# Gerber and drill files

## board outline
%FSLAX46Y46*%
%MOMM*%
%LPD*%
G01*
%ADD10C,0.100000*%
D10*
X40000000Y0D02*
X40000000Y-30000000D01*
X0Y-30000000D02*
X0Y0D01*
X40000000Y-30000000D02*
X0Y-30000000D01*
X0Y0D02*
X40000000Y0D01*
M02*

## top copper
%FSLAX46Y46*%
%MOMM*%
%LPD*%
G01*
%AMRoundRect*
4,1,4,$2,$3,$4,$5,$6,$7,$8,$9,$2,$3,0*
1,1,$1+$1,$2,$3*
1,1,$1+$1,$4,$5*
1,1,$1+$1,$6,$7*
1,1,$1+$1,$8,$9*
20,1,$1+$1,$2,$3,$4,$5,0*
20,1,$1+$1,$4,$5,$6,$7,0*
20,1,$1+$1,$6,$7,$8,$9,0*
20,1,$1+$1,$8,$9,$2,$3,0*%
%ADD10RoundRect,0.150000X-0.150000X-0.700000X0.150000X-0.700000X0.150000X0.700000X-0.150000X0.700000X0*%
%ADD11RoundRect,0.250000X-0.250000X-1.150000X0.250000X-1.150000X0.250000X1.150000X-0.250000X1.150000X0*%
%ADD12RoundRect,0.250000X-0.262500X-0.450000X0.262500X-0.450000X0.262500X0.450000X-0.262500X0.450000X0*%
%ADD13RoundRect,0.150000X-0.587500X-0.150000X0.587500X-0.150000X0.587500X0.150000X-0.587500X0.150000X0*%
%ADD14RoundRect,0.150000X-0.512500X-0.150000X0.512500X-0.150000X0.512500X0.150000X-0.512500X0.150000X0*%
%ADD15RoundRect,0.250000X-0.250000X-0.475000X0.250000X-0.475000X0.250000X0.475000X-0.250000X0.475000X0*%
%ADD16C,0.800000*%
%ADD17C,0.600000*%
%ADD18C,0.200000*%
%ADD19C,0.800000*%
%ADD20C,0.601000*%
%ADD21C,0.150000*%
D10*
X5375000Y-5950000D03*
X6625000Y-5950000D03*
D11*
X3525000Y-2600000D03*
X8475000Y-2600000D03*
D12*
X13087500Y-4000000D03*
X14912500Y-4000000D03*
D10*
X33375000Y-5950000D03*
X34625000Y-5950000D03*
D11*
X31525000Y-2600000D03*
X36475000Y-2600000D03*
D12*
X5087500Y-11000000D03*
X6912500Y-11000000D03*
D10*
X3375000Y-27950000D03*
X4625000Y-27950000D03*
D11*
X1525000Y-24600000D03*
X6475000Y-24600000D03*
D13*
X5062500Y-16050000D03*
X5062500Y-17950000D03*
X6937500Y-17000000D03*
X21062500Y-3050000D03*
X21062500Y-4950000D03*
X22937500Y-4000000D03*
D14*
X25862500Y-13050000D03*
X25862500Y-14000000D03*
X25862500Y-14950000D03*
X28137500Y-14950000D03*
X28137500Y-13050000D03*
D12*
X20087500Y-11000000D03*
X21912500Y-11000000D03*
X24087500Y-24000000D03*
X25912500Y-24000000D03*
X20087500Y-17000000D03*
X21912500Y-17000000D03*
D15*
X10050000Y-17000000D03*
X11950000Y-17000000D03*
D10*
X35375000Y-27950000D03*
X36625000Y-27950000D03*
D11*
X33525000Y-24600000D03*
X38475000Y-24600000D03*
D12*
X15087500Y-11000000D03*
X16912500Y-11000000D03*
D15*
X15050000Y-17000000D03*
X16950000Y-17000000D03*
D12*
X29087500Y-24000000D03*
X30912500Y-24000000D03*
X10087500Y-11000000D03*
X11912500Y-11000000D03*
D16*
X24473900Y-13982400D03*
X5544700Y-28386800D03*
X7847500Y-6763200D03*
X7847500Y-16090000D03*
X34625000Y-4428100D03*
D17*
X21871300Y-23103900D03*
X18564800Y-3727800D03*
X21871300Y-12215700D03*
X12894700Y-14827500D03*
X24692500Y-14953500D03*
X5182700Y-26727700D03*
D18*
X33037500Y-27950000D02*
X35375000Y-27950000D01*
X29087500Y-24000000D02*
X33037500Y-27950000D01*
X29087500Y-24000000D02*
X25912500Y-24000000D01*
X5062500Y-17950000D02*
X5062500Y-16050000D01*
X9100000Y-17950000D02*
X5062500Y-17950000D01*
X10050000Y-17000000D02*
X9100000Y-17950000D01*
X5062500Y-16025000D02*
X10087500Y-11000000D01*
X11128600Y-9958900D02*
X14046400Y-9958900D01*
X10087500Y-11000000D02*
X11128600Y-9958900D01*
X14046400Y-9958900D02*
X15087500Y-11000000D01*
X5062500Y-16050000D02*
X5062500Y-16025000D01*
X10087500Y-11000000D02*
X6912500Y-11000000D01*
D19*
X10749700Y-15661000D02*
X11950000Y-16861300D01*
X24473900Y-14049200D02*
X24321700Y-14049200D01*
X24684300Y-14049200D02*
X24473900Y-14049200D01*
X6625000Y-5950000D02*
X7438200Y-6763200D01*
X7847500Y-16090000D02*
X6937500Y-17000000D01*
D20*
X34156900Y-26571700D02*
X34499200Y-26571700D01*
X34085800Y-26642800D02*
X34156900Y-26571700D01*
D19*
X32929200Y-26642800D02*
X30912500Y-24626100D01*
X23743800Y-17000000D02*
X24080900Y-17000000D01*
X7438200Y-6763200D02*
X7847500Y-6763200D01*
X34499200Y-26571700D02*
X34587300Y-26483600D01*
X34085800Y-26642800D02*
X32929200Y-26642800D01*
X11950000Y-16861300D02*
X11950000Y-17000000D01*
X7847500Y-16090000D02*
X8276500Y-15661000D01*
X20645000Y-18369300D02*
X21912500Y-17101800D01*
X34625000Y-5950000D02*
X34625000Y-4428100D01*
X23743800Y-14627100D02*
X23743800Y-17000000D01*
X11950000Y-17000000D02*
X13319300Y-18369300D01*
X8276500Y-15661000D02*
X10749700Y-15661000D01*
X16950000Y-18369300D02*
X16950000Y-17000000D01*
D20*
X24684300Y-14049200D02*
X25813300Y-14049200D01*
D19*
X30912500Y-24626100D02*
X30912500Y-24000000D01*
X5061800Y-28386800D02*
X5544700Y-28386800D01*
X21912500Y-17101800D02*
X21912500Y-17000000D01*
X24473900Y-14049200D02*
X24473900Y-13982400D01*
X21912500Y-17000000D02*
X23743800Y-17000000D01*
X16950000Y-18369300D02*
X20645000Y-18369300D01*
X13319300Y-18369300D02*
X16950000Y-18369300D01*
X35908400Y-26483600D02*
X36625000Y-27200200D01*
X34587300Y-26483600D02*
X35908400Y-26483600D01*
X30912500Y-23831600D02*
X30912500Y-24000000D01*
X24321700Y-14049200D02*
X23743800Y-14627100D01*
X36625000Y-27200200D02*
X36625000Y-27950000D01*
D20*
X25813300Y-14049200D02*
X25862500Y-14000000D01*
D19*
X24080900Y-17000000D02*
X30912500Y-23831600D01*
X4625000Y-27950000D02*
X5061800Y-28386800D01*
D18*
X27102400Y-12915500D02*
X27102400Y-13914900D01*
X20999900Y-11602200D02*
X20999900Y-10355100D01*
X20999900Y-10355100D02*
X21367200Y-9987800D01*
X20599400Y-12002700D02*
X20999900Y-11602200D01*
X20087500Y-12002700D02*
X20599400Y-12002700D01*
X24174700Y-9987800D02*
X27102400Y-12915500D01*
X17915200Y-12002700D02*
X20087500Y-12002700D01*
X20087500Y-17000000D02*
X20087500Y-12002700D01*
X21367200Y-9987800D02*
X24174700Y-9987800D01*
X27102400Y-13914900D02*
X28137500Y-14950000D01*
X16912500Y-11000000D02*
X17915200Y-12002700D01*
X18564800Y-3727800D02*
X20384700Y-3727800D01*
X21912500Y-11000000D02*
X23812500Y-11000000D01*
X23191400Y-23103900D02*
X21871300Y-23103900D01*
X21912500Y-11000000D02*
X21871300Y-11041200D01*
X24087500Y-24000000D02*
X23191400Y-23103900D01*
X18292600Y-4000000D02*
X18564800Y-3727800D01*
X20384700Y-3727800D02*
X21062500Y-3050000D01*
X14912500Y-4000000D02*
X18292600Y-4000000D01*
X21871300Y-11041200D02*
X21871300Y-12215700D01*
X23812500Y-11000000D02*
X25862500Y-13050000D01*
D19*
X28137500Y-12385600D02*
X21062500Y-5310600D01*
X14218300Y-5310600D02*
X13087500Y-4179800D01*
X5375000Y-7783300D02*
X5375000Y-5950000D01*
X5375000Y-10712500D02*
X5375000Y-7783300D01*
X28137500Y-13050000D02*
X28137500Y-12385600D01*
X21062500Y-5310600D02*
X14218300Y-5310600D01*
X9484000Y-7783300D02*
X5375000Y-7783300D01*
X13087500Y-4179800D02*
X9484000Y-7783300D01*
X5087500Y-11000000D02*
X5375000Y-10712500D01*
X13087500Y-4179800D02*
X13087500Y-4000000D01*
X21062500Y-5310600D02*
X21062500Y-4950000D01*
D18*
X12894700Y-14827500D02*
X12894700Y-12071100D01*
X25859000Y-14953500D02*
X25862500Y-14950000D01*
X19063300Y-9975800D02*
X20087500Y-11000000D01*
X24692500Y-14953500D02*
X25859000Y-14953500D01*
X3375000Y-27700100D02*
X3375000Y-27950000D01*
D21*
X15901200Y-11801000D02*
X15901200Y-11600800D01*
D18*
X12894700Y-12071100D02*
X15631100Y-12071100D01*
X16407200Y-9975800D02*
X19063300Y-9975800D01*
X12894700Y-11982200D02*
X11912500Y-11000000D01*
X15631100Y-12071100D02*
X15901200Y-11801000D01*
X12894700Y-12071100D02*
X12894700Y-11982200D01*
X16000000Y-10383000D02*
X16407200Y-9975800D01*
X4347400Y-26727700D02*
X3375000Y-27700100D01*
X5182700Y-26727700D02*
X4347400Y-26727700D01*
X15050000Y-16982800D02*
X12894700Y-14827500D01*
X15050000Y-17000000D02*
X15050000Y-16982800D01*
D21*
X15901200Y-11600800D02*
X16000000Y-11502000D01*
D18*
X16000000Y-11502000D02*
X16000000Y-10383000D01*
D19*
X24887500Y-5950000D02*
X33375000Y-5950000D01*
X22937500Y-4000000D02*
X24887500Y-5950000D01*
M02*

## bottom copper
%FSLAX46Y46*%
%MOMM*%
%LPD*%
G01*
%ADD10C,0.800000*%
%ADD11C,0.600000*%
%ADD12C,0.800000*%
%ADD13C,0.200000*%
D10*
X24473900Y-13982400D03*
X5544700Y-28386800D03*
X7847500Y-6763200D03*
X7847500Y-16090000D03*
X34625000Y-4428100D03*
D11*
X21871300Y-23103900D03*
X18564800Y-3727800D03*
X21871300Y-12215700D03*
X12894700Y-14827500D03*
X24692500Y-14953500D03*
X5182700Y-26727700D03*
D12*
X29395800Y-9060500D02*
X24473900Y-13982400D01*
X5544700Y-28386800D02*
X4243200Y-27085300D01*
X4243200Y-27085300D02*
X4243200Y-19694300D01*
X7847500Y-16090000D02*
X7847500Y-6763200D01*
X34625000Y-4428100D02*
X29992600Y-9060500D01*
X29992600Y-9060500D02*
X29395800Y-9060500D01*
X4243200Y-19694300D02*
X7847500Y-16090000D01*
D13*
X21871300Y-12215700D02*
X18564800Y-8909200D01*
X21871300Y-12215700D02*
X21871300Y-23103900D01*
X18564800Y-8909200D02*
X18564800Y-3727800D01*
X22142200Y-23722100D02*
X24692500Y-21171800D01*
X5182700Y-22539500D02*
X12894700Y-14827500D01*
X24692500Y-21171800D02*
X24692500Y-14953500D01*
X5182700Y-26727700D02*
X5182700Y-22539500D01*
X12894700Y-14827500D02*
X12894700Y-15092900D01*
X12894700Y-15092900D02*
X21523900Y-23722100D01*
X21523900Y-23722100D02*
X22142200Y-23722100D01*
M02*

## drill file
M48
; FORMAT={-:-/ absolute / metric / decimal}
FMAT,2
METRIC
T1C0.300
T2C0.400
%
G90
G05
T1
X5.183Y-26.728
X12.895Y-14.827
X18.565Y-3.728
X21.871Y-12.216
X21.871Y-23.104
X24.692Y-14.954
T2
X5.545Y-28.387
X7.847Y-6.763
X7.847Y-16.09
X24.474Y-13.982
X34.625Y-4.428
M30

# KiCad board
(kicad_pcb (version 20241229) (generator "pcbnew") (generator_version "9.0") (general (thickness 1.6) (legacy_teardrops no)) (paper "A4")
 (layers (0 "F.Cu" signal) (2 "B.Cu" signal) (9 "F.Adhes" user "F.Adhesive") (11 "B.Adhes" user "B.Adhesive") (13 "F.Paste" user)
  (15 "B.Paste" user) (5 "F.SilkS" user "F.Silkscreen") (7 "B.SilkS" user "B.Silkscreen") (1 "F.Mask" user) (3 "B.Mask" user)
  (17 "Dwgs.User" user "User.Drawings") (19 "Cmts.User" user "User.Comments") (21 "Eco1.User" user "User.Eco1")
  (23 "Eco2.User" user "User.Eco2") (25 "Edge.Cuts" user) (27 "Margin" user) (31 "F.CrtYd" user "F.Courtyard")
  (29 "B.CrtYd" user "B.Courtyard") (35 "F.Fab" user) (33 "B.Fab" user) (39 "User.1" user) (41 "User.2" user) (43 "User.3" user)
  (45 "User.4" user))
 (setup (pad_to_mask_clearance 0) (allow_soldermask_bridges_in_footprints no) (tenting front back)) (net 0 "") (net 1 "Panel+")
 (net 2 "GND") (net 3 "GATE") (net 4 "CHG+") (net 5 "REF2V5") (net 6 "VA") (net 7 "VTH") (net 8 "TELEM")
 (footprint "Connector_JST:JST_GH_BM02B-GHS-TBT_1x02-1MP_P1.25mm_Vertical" (layer "F.Cu") (at 6 4)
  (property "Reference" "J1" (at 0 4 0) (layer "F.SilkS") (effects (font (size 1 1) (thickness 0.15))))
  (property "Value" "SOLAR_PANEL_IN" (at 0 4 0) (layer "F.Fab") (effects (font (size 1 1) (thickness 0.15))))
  (pad "1" smd roundrect (at -0.625 1.95) (size 0.6 1.7) (layers "F.Cu" "F.Mask" "F.Paste") (roundrect_rratio 0.25) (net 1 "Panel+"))
  (pad "2" smd roundrect (at 0.625 1.95) (size 0.6 1.7) (layers "F.Cu" "F.Mask" "F.Paste") (roundrect_rratio 0.25) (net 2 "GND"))
  (pad "MP" smd roundrect (at -2.475 -1.4) (size 1 2.8) (layers "F.Cu" "F.Mask" "F.Paste") (roundrect_rratio 0.25))
  (pad "MP" smd roundrect (at 2.475 -1.4) (size 1 2.8) (layers "F.Cu" "F.Mask" "F.Paste") (roundrect_rratio 0.25)))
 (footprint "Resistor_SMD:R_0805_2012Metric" (layer "F.Cu") (at 14 4)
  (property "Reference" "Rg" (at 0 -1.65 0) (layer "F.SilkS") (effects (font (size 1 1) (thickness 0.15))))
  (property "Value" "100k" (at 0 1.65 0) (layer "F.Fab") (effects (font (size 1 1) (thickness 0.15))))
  (pad "1" smd roundrect (at -0.9125 0) (size 1.025 1.4) (layers "F.Cu" "F.Mask" "F.Paste") (roundrect_rratio 0.243902) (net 1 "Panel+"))
  (pad "2" smd roundrect (at 0.9125 0) (size 1.025 1.4) (layers "F.Cu" "F.Mask" "F.Paste") (roundrect_rratio 0.243902) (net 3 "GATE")))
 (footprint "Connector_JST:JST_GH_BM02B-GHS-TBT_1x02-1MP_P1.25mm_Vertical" (layer "F.Cu") (at 34 4)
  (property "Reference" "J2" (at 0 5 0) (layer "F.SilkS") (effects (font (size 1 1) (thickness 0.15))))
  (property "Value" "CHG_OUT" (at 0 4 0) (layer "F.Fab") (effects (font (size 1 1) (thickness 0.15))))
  (pad "1" smd roundrect (at -0.625 1.95) (size 0.6 1.7) (layers "F.Cu" "F.Mask" "F.Paste") (roundrect_rratio 0.25) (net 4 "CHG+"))
  (pad "2" smd roundrect (at 0.625 1.95) (size 0.6 1.7) (layers "F.Cu" "F.Mask" "F.Paste") (roundrect_rratio 0.25) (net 2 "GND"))
  (pad "MP" smd roundrect (at -2.475 -1.4) (size 1 2.8) (layers "F.Cu" "F.Mask" "F.Paste") (roundrect_rratio 0.25))
  (pad "MP" smd roundrect (at 2.475 -1.4) (size 1 2.8) (layers "F.Cu" "F.Mask" "F.Paste") (roundrect_rratio 0.25)))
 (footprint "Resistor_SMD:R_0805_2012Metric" (layer "F.Cu") (at 6 11)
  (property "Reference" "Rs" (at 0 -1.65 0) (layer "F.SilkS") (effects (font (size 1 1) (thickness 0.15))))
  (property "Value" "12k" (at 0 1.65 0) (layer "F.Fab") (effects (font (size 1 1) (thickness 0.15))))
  (pad "1" smd roundrect (at -0.9125 0) (size 1.025 1.4) (layers "F.Cu" "F.Mask" "F.Paste") (roundrect_rratio 0.243902) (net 1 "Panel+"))
  (pad "2" smd roundrect (at 0.9125 0) (size 1.025 1.4) (layers "F.Cu" "F.Mask" "F.Paste") (roundrect_rratio 0.243902) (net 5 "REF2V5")))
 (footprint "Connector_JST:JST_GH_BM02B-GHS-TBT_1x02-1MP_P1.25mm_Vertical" (layer "F.Cu") (at 4 26)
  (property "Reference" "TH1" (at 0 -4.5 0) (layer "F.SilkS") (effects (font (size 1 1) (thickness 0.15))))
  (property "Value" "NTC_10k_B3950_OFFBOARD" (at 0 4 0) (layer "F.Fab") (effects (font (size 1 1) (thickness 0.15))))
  (pad "1" smd roundrect (at -0.625 1.95) (size 0.6 1.7) (layers "F.Cu" "F.Mask" "F.Paste") (roundrect_rratio 0.25) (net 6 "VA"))
  (pad "2" smd roundrect (at 0.625 1.95) (size 0.6 1.7) (layers "F.Cu" "F.Mask" "F.Paste") (roundrect_rratio 0.25) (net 2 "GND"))
  (pad "MP" smd roundrect (at -2.475 -1.4) (size 1 2.8) (layers "F.Cu" "F.Mask" "F.Paste") (roundrect_rratio 0.25))
  (pad "MP" smd roundrect (at 2.475 -1.4) (size 1 2.8) (layers "F.Cu" "F.Mask" "F.Paste") (roundrect_rratio 0.25)))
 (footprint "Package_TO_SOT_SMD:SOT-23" (layer "F.Cu") (at 6 17)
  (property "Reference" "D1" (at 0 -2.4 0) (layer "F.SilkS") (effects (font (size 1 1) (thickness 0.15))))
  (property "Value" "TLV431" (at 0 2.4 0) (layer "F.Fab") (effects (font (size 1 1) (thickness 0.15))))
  (pad "1" smd roundrect (at -0.9375 -0.95) (size 1.475 0.6) (layers "F.Cu" "F.Mask" "F.Paste") (roundrect_rratio 0.25) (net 5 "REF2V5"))
  (pad "2" smd roundrect (at -0.9375 0.95) (size 1.475 0.6) (layers "F.Cu" "F.Mask" "F.Paste") (roundrect_rratio 0.25) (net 5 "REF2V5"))
  (pad "3" smd roundrect (at 0.9375 0) (size 1.475 0.6) (layers "F.Cu" "F.Mask" "F.Paste") (roundrect_rratio 0.25) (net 2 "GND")))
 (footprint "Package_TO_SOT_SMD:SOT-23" (layer "F.Cu") (at 22 4)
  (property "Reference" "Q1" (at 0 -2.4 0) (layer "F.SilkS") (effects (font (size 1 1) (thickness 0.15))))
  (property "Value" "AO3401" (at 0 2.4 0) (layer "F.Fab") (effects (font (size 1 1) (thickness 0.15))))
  (pad "1" smd roundrect (at -0.9375 -0.95) (size 1.475 0.6) (layers "F.Cu" "F.Mask" "F.Paste") (roundrect_rratio 0.25) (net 3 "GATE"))
  (pad "2" smd roundrect (at -0.9375 0.95) (size 1.475 0.6) (layers "F.Cu" "F.Mask" "F.Paste") (roundrect_rratio 0.25) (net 1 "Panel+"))
  (pad "3" smd roundrect (at 0.9375 0) (size 1.475 0.6) (layers "F.Cu" "F.Mask" "F.Paste") (roundrect_rratio 0.25) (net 4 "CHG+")))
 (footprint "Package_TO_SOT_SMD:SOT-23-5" (layer "F.Cu") (at 27 14)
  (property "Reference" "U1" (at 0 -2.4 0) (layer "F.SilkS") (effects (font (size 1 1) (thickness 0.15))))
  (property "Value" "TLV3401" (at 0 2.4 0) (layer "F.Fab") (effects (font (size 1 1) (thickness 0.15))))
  (pad "1" smd roundrect (at -1.1375 -0.95) (size 1.325 0.6) (layers "F.Cu" "F.Mask" "F.Paste") (roundrect_rratio 0.25) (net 3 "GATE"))
  (pad "2" smd roundrect (at -1.1375 0) (size 1.325 0.6) (layers "F.Cu" "F.Mask" "F.Paste") (roundrect_rratio 0.25) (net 2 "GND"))
  (pad "3" smd roundrect (at -1.1375 0.95) (size 1.325 0.6) (layers "F.Cu" "F.Mask" "F.Paste") (roundrect_rratio 0.25) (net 6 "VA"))
  (pad "4" smd roundrect (at 1.1375 0.95) (size 1.325 0.6) (layers "F.Cu" "F.Mask" "F.Paste") (roundrect_rratio 0.25) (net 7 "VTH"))
  (pad "5" smd roundrect (at 1.1375 -0.95) (size 1.325 0.6) (layers "F.Cu" "F.Mask" "F.Paste") (roundrect_rratio 0.25) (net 1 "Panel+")))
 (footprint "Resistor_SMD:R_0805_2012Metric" (layer "F.Cu") (at 21 11)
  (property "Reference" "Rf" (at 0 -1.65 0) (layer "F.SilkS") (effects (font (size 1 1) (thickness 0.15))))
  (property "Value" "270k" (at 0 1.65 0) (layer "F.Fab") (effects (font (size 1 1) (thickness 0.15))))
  (pad "1" smd roundrect (at -0.9125 0) (size 1.025 1.4) (layers "F.Cu" "F.Mask" "F.Paste") (roundrect_rratio 0.243902) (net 6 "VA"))
  (pad "2" smd roundrect (at 0.9125 0) (size 1.025 1.4) (layers "F.Cu" "F.Mask" "F.Paste") (roundrect_rratio 0.243902) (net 3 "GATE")))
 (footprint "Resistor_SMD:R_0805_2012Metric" (layer "F.Cu") (at 25 24)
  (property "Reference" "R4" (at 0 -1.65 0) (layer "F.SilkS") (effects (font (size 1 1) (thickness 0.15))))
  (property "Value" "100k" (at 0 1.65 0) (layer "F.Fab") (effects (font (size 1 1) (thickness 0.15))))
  (pad "1" smd roundrect (at -0.9125 0) (size 1.025 1.4) (layers "F.Cu" "F.Mask" "F.Paste") (roundrect_rratio 0.243902) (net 3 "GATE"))
  (pad "2" smd roundrect (at 0.9125 0) (size 1.025 1.4) (layers "F.Cu" "F.Mask" "F.Paste") (roundrect_rratio 0.243902) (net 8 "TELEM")))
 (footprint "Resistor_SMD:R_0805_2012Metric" (layer "F.Cu") (at 21 17)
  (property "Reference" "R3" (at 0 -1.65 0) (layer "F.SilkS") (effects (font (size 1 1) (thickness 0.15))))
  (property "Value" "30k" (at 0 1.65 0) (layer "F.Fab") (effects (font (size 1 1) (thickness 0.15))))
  (pad "1" smd roundrect (at -0.9125 0) (size 1.025 1.4) (layers "F.Cu" "F.Mask" "F.Paste") (roundrect_rratio 0.243902) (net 7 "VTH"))
  (pad "2" smd roundrect (at 0.9125 0) (size 1.025 1.4) (layers "F.Cu" "F.Mask" "F.Paste") (roundrect_rratio 0.243902) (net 2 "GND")))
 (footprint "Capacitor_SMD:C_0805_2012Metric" (layer "F.Cu") (at 11 17)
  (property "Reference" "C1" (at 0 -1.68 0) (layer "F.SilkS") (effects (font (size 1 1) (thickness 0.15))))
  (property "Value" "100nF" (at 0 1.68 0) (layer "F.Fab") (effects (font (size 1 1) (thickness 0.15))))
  (pad "1" smd roundrect (at -0.95 0) (size 1 1.45) (layers "F.Cu" "F.Mask" "F.Paste") (roundrect_rratio 0.25) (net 5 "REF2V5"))
  (pad "2" smd roundrect (at 0.95 0) (size 1 1.45) (layers "F.Cu" "F.Mask" "F.Paste") (roundrect_rratio 0.25) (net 2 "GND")))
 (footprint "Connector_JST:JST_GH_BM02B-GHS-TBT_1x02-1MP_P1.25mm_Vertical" (layer "F.Cu") (at 36 26)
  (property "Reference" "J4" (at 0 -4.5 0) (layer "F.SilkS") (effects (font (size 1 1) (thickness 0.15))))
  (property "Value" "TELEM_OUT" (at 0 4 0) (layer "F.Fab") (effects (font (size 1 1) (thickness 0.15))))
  (pad "1" smd roundrect (at -0.625 1.95) (size 0.6 1.7) (layers "F.Cu" "F.Mask" "F.Paste") (roundrect_rratio 0.25) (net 8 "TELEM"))
  (pad "2" smd roundrect (at 0.625 1.95) (size 0.6 1.7) (layers "F.Cu" "F.Mask" "F.Paste") (roundrect_rratio 0.25) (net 2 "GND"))
  (pad "MP" smd roundrect (at -2.475 -1.4) (size 1 2.8) (layers "F.Cu" "F.Mask" "F.Paste") (roundrect_rratio 0.25))
  (pad "MP" smd roundrect (at 2.475 -1.4) (size 1 2.8) (layers "F.Cu" "F.Mask" "F.Paste") (roundrect_rratio 0.25)))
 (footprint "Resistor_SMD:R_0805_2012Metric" (layer "F.Cu") (at 16 11)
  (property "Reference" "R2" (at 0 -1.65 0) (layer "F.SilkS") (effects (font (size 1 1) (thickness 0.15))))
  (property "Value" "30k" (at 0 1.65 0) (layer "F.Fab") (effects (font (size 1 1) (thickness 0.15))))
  (pad "1" smd roundrect (at -0.9125 0) (size 1.025 1.4) (layers "F.Cu" "F.Mask" "F.Paste") (roundrect_rratio 0.243902) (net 5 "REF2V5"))
  (pad "2" smd roundrect (at 0.9125 0) (size 1.025 1.4) (layers "F.Cu" "F.Mask" "F.Paste") (roundrect_rratio 0.243902) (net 7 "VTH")))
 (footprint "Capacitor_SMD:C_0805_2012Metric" (layer "F.Cu") (at 16 17)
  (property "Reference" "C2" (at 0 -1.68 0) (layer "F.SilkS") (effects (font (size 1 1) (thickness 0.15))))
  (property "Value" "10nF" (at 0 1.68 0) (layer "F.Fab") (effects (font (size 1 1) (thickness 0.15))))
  (pad "1" smd roundrect (at -0.95 0) (size 1 1.45) (layers "F.Cu" "F.Mask" "F.Paste") (roundrect_rratio 0.25) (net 6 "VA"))
  (pad "2" smd roundrect (at 0.95 0) (size 1 1.45) (layers "F.Cu" "F.Mask" "F.Paste") (roundrect_rratio 0.25) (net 2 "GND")))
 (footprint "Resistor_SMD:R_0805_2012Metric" (layer "F.Cu") (at 30 24)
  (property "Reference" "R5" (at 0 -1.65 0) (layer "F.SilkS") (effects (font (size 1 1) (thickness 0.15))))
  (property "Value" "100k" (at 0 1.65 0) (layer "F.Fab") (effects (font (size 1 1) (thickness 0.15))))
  (pad "1" smd roundrect (at -0.9125 0) (size 1.025 1.4) (layers "F.Cu" "F.Mask" "F.Paste") (roundrect_rratio 0.243902) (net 8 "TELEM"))
  (pad "2" smd roundrect (at 0.9125 0) (size 1.025 1.4) (layers "F.Cu" "F.Mask" "F.Paste") (roundrect_rratio 0.243902) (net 2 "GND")))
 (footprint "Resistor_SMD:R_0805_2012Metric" (layer "F.Cu") (at 11 11)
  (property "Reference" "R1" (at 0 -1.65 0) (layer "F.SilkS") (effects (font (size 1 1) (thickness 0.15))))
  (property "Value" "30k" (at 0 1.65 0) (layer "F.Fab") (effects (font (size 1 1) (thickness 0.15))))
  (pad "1" smd roundrect (at -0.9125 0) (size 1.025 1.4) (layers "F.Cu" "F.Mask" "F.Paste") (roundrect_rratio 0.243902) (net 5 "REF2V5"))
  (pad "2" smd roundrect (at 0.9125 0) (size 1.025 1.4) (layers "F.Cu" "F.Mask" "F.Paste") (roundrect_rratio 0.243902) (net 6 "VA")))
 (gr_line (start 40 0) (end 40 30) (stroke (width 0.1) (type default)) (layer "Edge.Cuts"))
 (gr_line (start 0 30) (end 0 0) (stroke (width 0.1) (type default)) (layer "Edge.Cuts"))
 (gr_line (start 40 30) (end 0 30) (stroke (width 0.1) (type default)) (layer "Edge.Cuts"))
 (gr_line (start 0 0) (end 40 0) (stroke (width 0.1) (type default)) (layer "Edge.Cuts"))
 (segment (start 33.0375 27.95) (end 35.375 27.95) (width 0.2) (layer "F.Cu") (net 8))
 (segment (start 29.0875 24) (end 33.0375 27.95) (width 0.2) (layer "F.Cu") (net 8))
 (segment (start 29.0875 24) (end 25.9125 24) (width 0.2) (layer "F.Cu") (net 8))
 (segment (start 5.0625 17.95) (end 5.0625 16.05) (width 0.2) (layer "F.Cu") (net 5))
 (segment (start 9.1 17.95) (end 5.0625 17.95) (width 0.2) (layer "F.Cu") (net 5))
 (segment (start 10.05 17) (end 9.1 17.95) (width 0.2) (layer "F.Cu") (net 5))
 (segment (start 5.0625 16.025) (end 10.0875 11) (width 0.2) (layer "F.Cu") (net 5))
 (segment (start 11.1286 9.9589) (end 14.0464 9.9589) (width 0.2) (layer "F.Cu") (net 5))
 (segment (start 10.0875 11) (end 11.1286 9.9589) (width 0.2) (layer "F.Cu") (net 5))
 (segment (start 14.0464 9.9589) (end 15.0875 11) (width 0.2) (layer "F.Cu") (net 5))
 (segment (start 5.0625 16.05) (end 5.0625 16.025) (width 0.2) (layer "F.Cu") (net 5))
 (segment (start 10.0875 11) (end 6.9125 11) (width 0.2) (layer "F.Cu") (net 5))
 (segment (start 10.7497 15.661) (end 11.95 16.8613) (width 0.8) (layer "F.Cu") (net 2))
 (segment (start 24.4739 14.0492) (end 24.3217 14.0492) (width 0.8) (layer "F.Cu") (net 2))
 (segment (start 24.6843 14.0492) (end 24.4739 14.0492) (width 0.8) (layer "F.Cu") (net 2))
 (segment (start 6.625 5.95) (end 7.4382 6.7632) (width 0.8) (layer "F.Cu") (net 2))
 (segment (start 7.8475 16.09) (end 6.9375 17) (width 0.8) (layer "F.Cu") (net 2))
 (segment (start 34.1569 26.5717) (end 34.4992 26.5717) (width 0.601) (layer "F.Cu") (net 2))
 (segment (start 34.0858 26.6428) (end 34.1569 26.5717) (width 0.601) (layer "F.Cu") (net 2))
 (segment (start 32.9292 26.6428) (end 30.9125 24.6261) (width 0.8) (layer "F.Cu") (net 2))
 (segment (start 23.7438 17) (end 24.0809 17) (width 0.8) (layer "F.Cu") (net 2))
 (segment (start 7.4382 6.7632) (end 7.8475 6.7632) (width 0.8) (layer "F.Cu") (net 2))
 (segment (start 34.4992 26.5717) (end 34.5873 26.4836) (width 0.8) (layer "F.Cu") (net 2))
 (segment (start 34.0858 26.6428) (end 32.9292 26.6428) (width 0.8) (layer "F.Cu") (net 2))
 (segment (start 11.95 16.8613) (end 11.95 17) (width 0.8) (layer "F.Cu") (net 2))
 (segment (start 7.8475 16.09) (end 8.2765 15.661) (width 0.8) (layer "F.Cu") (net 2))
 (segment (start 20.645 18.3693) (end 21.9125 17.1018) (width 0.8) (layer "F.Cu") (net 2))
 (segment (start 34.625 5.95) (end 34.625 4.4281) (width 0.8) (layer "F.Cu") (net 2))
 (segment (start 23.7438 14.6271) (end 23.7438 17) (width 0.8) (layer "F.Cu") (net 2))
 (segment (start 11.95 17) (end 13.3193 18.3693) (width 0.8) (layer "F.Cu") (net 2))
 (segment (start 8.2765 15.661) (end 10.7497 15.661) (width 0.8) (layer "F.Cu") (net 2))
 (segment (start 16.95 18.3693) (end 16.95 17) (width 0.8) (layer "F.Cu") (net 2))
 (segment (start 24.6843 14.0492) (end 25.8133 14.0492) (width 0.601) (layer "F.Cu") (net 2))
 (segment (start 30.9125 24.6261) (end 30.9125 24) (width 0.8) (layer "F.Cu") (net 2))
 (segment (start 5.0618 28.3868) (end 5.5447 28.3868) (width 0.8) (layer "F.Cu") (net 2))
 (segment (start 21.9125 17.1018) (end 21.9125 17) (width 0.8) (layer "F.Cu") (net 2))
 (segment (start 24.4739 14.0492) (end 24.4739 13.9824) (width 0.8) (layer "F.Cu") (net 2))
 (segment (start 21.9125 17) (end 23.7438 17) (width 0.8) (layer "F.Cu") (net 2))
 (segment (start 16.95 18.3693) (end 20.645 18.3693) (width 0.8) (layer "F.Cu") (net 2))
 (segment (start 13.3193 18.3693) (end 16.95 18.3693) (width 0.8) (layer "F.Cu") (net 2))
 (segment (start 35.9084 26.4836) (end 36.625 27.2002) (width 0.8) (layer "F.Cu") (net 2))
 (segment (start 34.5873 26.4836) (end 35.9084 26.4836) (width 0.8) (layer "F.Cu") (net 2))
 (segment (start 30.9125 23.8316) (end 30.9125 24) (width 0.8) (layer "F.Cu") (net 2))
 (segment (start 24.3217 14.0492) (end 23.7438 14.6271) (width 0.8) (layer "F.Cu") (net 2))
 (segment (start 36.625 27.2002) (end 36.625 27.95) (width 0.8) (layer "F.Cu") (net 2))
 (segment (start 25.8133 14.0492) (end 25.8625 14) (width 0.601) (layer "F.Cu") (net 2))
 (segment (start 24.0809 17) (end 30.9125 23.8316) (width 0.8) (layer "F.Cu") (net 2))
 (segment (start 4.625 27.95) (end 5.0618 28.3868) (width 0.8) (layer "F.Cu") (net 2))
 (via (at 24.4739 13.9824) (size 0.8) (drill 0.4) (layers "F.Cu" "B.Cu") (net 2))
 (via (at 5.5447 28.3868) (size 0.8) (drill 0.4) (layers "F.Cu" "B.Cu") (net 2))
 (via (at 7.8475 6.7632) (size 0.8) (drill 0.4) (layers "F.Cu" "B.Cu") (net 2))
 (via (at 7.8475 16.09) (size 0.8) (drill 0.4) (layers "F.Cu" "B.Cu") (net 2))
 (via (at 34.625 4.4281) (size 0.8) (drill 0.4) (layers "F.Cu" "B.Cu") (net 2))
 (segment (start 29.3958 9.0605) (end 24.4739 13.9824) (width 0.8) (layer "B.Cu") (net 2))
 (segment (start 5.5447 28.3868) (end 4.2432 27.0853) (width 0.8) (layer "B.Cu") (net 2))
 (segment (start 4.2432 27.0853) (end 4.2432 19.6943) (width 0.8) (layer "B.Cu") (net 2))
 (segment (start 7.8475 16.09) (end 7.8475 6.7632) (width 0.8) (layer "B.Cu") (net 2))
 (segment (start 34.625 4.4281) (end 29.9926 9.0605) (width 0.8) (layer "B.Cu") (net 2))
 (segment (start 29.9926 9.0605) (end 29.3958 9.0605) (width 0.8) (layer "B.Cu") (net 2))
 (segment (start 4.2432 19.6943) (end 7.8475 16.09) (width 0.8) (layer "B.Cu") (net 2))
 (segment (start 27.1024 12.9155) (end 27.1024 13.9149) (width 0.2) (layer "F.Cu") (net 7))
 (segment (start 20.9999 11.6022) (end 20.9999 10.3551) (width 0.2) (layer "F.Cu") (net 7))
 (segment (start 20.9999 10.3551) (end 21.3672 9.9878) (width 0.2) (layer "F.Cu") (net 7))
 (segment (start 20.5994 12.0027) (end 20.9999 11.6022) (width 0.2) (layer "F.Cu") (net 7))
 (segment (start 20.0875 12.0027) (end 20.5994 12.0027) (width 0.2) (layer "F.Cu") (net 7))
 (segment (start 24.1747 9.9878) (end 27.1024 12.9155) (width 0.2) (layer "F.Cu") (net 7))
 (segment (start 17.9152 12.0027) (end 20.0875 12.0027) (width 0.2) (layer "F.Cu") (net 7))
 (segment (start 20.0875 17) (end 20.0875 12.0027) (width 0.2) (layer "F.Cu") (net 7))
 (segment (start 21.3672 9.9878) (end 24.1747 9.9878) (width 0.2) (layer "F.Cu") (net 7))
 (segment (start 27.1024 13.9149) (end 28.1375 14.95) (width 0.2) (layer "F.Cu") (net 7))
 (segment (start 16.9125 11) (end 17.9152 12.0027) (width 0.2) (layer "F.Cu") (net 7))
 (segment (start 18.5648 3.7278) (end 20.3847 3.7278) (width 0.2) (layer "F.Cu") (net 3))
 (segment (start 21.9125 11) (end 23.8125 11) (width 0.2) (layer "F.Cu") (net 3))
 (segment (start 23.1914 23.1039) (end 21.8713 23.1039) (width 0.2) (layer "F.Cu") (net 3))
 (segment (start 21.9125 11) (end 21.8713 11.0412) (width 0.2) (layer "F.Cu") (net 3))
 (segment (start 24.0875 24) (end 23.1914 23.1039) (width 0.2) (layer "F.Cu") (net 3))
 (segment (start 18.2926 4) (end 18.5648 3.7278) (width 0.2) (layer "F.Cu") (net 3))
 (segment (start 20.3847 3.7278) (end 21.0625 3.05) (width 0.2) (layer "F.Cu") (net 3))
 (segment (start 14.9125 4) (end 18.2926 4) (width 0.2) (layer "F.Cu") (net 3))
 (segment (start 21.8713 11.0412) (end 21.8713 12.2157) (width 0.2) (layer "F.Cu") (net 3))
 (segment (start 23.8125 11) (end 25.8625 13.05) (width 0.2) (layer "F.Cu") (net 3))
 (via (at 21.8713 23.1039) (size 0.6) (drill 0.3) (layers "F.Cu" "B.Cu") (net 3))
 (via (at 18.5648 3.7278) (size 0.6) (drill 0.3) (layers "F.Cu" "B.Cu") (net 3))
 (via (at 21.8713 12.2157) (size 0.6) (drill 0.3) (layers "F.Cu" "B.Cu") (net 3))
 (segment (start 21.8713 12.2157) (end 18.5648 8.9092) (width 0.2) (layer "B.Cu") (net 3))
 (segment (start 21.8713 12.2157) (end 21.8713 23.1039) (width 0.2) (layer "B.Cu") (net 3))
 (segment (start 18.5648 8.9092) (end 18.5648 3.7278) (width 0.2) (layer "B.Cu") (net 3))
 (segment (start 28.1375 12.3856) (end 21.0625 5.3106) (width 0.8) (layer "F.Cu") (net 1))
 (segment (start 14.2183 5.3106) (end 13.0875 4.1798) (width 0.8) (layer "F.Cu") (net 1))
 (segment (start 5.375 7.7833) (end 5.375 5.95) (width 0.8) (layer "F.Cu") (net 1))
 (segment (start 5.375 10.7125) (end 5.375 7.7833) (width 0.8) (layer "F.Cu") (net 1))
 (segment (start 28.1375 13.05) (end 28.1375 12.3856) (width 0.8) (layer "F.Cu") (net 1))
 (segment (start 21.0625 5.3106) (end 14.2183 5.3106) (width 0.8) (layer "F.Cu") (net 1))
 (segment (start 9.484 7.7833) (end 5.375 7.7833) (width 0.8) (layer "F.Cu") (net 1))
 (segment (start 13.0875 4.1798) (end 9.484 7.7833) (width 0.8) (layer "F.Cu") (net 1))
 (segment (start 5.0875 11) (end 5.375 10.7125) (width 0.8) (layer "F.Cu") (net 1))
 (segment (start 13.0875 4.1798) (end 13.0875 4) (width 0.8) (layer "F.Cu") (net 1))
 (segment (start 21.0625 5.3106) (end 21.0625 4.95) (width 0.8) (layer "F.Cu") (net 1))
 (segment (start 12.8947 14.8275) (end 12.8947 12.0711) (width 0.2) (layer "F.Cu") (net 6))
 (segment (start 25.859 14.9535) (end 25.8625 14.95) (width 0.2) (layer "F.Cu") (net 6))
 (segment (start 19.0633 9.9758) (end 20.0875 11) (width 0.2) (layer "F.Cu") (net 6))
 (segment (start 24.6925 14.9535) (end 25.859 14.9535) (width 0.2) (layer "F.Cu") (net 6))
 (segment (start 3.375 27.7001) (end 3.375 27.95) (width 0.2) (layer "F.Cu") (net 6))
 (segment (start 15.9012 11.801) (end 15.9012 11.6008) (width 0.15) (layer "F.Cu") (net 6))
 (segment (start 12.8947 12.0711) (end 15.6311 12.0711) (width 0.2) (layer "F.Cu") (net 6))
 (segment (start 16.4072 9.9758) (end 19.0633 9.9758) (width 0.2) (layer "F.Cu") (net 6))
 (segment (start 12.8947 11.9822) (end 11.9125 11) (width 0.2) (layer "F.Cu") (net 6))
 (segment (start 15.6311 12.0711) (end 15.9012 11.801) (width 0.2) (layer "F.Cu") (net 6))
 (segment (start 12.8947 12.0711) (end 12.8947 11.9822) (width 0.2) (layer "F.Cu") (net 6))
 (segment (start 16 10.383) (end 16.4072 9.9758) (width 0.2) (layer "F.Cu") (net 6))
 (segment (start 4.3474 26.7277) (end 3.375 27.7001) (width 0.2) (layer "F.Cu") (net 6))
 (segment (start 5.1827 26.7277) (end 4.3474 26.7277) (width 0.2) (layer "F.Cu") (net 6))
 (segment (start 15.05 16.9828) (end 12.8947 14.8275) (width 0.2) (layer "F.Cu") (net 6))
 (segment (start 15.05 17) (end 15.05 16.9828) (width 0.2) (layer "F.Cu") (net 6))
 (segment (start 15.9012 11.6008) (end 16 11.502) (width 0.15) (layer "F.Cu") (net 6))
 (segment (start 16 11.502) (end 16 10.383) (width 0.2) (layer "F.Cu") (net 6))
 (via (at 12.8947 14.8275) (size 0.6) (drill 0.3) (layers "F.Cu" "B.Cu") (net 6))
 (via (at 24.6925 14.9535) (size 0.6) (drill 0.3) (layers "F.Cu" "B.Cu") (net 6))
 (via (at 5.1827 26.7277) (size 0.6) (drill 0.3) (layers "F.Cu" "B.Cu") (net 6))
 (segment (start 22.1422 23.7221) (end 24.6925 21.1718) (width 0.2) (layer "B.Cu") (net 6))
 (segment (start 5.1827 22.5395) (end 12.8947 14.8275) (width 0.2) (layer "B.Cu") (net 6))
 (segment (start 24.6925 21.1718) (end 24.6925 14.9535) (width 0.2) (layer "B.Cu") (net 6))
 (segment (start 5.1827 26.7277) (end 5.1827 22.5395) (width 0.2) (layer "B.Cu") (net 6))
 (segment (start 12.8947 14.8275) (end 12.8947 15.0929) (width 0.2) (layer "B.Cu") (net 6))
 (segment (start 12.8947 15.0929) (end 21.5239 23.7221) (width 0.2) (layer "B.Cu") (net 6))
 (segment (start 21.5239 23.7221) (end 22.1422 23.7221) (width 0.2) (layer "B.Cu") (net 6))
 (segment (start 24.8875 5.95) (end 33.375 5.95) (width 0.8) (layer "F.Cu") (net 4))
 (segment (start 22.9375 4) (end 24.8875 5.95) (width 0.8) (layer "F.Cu") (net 4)))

